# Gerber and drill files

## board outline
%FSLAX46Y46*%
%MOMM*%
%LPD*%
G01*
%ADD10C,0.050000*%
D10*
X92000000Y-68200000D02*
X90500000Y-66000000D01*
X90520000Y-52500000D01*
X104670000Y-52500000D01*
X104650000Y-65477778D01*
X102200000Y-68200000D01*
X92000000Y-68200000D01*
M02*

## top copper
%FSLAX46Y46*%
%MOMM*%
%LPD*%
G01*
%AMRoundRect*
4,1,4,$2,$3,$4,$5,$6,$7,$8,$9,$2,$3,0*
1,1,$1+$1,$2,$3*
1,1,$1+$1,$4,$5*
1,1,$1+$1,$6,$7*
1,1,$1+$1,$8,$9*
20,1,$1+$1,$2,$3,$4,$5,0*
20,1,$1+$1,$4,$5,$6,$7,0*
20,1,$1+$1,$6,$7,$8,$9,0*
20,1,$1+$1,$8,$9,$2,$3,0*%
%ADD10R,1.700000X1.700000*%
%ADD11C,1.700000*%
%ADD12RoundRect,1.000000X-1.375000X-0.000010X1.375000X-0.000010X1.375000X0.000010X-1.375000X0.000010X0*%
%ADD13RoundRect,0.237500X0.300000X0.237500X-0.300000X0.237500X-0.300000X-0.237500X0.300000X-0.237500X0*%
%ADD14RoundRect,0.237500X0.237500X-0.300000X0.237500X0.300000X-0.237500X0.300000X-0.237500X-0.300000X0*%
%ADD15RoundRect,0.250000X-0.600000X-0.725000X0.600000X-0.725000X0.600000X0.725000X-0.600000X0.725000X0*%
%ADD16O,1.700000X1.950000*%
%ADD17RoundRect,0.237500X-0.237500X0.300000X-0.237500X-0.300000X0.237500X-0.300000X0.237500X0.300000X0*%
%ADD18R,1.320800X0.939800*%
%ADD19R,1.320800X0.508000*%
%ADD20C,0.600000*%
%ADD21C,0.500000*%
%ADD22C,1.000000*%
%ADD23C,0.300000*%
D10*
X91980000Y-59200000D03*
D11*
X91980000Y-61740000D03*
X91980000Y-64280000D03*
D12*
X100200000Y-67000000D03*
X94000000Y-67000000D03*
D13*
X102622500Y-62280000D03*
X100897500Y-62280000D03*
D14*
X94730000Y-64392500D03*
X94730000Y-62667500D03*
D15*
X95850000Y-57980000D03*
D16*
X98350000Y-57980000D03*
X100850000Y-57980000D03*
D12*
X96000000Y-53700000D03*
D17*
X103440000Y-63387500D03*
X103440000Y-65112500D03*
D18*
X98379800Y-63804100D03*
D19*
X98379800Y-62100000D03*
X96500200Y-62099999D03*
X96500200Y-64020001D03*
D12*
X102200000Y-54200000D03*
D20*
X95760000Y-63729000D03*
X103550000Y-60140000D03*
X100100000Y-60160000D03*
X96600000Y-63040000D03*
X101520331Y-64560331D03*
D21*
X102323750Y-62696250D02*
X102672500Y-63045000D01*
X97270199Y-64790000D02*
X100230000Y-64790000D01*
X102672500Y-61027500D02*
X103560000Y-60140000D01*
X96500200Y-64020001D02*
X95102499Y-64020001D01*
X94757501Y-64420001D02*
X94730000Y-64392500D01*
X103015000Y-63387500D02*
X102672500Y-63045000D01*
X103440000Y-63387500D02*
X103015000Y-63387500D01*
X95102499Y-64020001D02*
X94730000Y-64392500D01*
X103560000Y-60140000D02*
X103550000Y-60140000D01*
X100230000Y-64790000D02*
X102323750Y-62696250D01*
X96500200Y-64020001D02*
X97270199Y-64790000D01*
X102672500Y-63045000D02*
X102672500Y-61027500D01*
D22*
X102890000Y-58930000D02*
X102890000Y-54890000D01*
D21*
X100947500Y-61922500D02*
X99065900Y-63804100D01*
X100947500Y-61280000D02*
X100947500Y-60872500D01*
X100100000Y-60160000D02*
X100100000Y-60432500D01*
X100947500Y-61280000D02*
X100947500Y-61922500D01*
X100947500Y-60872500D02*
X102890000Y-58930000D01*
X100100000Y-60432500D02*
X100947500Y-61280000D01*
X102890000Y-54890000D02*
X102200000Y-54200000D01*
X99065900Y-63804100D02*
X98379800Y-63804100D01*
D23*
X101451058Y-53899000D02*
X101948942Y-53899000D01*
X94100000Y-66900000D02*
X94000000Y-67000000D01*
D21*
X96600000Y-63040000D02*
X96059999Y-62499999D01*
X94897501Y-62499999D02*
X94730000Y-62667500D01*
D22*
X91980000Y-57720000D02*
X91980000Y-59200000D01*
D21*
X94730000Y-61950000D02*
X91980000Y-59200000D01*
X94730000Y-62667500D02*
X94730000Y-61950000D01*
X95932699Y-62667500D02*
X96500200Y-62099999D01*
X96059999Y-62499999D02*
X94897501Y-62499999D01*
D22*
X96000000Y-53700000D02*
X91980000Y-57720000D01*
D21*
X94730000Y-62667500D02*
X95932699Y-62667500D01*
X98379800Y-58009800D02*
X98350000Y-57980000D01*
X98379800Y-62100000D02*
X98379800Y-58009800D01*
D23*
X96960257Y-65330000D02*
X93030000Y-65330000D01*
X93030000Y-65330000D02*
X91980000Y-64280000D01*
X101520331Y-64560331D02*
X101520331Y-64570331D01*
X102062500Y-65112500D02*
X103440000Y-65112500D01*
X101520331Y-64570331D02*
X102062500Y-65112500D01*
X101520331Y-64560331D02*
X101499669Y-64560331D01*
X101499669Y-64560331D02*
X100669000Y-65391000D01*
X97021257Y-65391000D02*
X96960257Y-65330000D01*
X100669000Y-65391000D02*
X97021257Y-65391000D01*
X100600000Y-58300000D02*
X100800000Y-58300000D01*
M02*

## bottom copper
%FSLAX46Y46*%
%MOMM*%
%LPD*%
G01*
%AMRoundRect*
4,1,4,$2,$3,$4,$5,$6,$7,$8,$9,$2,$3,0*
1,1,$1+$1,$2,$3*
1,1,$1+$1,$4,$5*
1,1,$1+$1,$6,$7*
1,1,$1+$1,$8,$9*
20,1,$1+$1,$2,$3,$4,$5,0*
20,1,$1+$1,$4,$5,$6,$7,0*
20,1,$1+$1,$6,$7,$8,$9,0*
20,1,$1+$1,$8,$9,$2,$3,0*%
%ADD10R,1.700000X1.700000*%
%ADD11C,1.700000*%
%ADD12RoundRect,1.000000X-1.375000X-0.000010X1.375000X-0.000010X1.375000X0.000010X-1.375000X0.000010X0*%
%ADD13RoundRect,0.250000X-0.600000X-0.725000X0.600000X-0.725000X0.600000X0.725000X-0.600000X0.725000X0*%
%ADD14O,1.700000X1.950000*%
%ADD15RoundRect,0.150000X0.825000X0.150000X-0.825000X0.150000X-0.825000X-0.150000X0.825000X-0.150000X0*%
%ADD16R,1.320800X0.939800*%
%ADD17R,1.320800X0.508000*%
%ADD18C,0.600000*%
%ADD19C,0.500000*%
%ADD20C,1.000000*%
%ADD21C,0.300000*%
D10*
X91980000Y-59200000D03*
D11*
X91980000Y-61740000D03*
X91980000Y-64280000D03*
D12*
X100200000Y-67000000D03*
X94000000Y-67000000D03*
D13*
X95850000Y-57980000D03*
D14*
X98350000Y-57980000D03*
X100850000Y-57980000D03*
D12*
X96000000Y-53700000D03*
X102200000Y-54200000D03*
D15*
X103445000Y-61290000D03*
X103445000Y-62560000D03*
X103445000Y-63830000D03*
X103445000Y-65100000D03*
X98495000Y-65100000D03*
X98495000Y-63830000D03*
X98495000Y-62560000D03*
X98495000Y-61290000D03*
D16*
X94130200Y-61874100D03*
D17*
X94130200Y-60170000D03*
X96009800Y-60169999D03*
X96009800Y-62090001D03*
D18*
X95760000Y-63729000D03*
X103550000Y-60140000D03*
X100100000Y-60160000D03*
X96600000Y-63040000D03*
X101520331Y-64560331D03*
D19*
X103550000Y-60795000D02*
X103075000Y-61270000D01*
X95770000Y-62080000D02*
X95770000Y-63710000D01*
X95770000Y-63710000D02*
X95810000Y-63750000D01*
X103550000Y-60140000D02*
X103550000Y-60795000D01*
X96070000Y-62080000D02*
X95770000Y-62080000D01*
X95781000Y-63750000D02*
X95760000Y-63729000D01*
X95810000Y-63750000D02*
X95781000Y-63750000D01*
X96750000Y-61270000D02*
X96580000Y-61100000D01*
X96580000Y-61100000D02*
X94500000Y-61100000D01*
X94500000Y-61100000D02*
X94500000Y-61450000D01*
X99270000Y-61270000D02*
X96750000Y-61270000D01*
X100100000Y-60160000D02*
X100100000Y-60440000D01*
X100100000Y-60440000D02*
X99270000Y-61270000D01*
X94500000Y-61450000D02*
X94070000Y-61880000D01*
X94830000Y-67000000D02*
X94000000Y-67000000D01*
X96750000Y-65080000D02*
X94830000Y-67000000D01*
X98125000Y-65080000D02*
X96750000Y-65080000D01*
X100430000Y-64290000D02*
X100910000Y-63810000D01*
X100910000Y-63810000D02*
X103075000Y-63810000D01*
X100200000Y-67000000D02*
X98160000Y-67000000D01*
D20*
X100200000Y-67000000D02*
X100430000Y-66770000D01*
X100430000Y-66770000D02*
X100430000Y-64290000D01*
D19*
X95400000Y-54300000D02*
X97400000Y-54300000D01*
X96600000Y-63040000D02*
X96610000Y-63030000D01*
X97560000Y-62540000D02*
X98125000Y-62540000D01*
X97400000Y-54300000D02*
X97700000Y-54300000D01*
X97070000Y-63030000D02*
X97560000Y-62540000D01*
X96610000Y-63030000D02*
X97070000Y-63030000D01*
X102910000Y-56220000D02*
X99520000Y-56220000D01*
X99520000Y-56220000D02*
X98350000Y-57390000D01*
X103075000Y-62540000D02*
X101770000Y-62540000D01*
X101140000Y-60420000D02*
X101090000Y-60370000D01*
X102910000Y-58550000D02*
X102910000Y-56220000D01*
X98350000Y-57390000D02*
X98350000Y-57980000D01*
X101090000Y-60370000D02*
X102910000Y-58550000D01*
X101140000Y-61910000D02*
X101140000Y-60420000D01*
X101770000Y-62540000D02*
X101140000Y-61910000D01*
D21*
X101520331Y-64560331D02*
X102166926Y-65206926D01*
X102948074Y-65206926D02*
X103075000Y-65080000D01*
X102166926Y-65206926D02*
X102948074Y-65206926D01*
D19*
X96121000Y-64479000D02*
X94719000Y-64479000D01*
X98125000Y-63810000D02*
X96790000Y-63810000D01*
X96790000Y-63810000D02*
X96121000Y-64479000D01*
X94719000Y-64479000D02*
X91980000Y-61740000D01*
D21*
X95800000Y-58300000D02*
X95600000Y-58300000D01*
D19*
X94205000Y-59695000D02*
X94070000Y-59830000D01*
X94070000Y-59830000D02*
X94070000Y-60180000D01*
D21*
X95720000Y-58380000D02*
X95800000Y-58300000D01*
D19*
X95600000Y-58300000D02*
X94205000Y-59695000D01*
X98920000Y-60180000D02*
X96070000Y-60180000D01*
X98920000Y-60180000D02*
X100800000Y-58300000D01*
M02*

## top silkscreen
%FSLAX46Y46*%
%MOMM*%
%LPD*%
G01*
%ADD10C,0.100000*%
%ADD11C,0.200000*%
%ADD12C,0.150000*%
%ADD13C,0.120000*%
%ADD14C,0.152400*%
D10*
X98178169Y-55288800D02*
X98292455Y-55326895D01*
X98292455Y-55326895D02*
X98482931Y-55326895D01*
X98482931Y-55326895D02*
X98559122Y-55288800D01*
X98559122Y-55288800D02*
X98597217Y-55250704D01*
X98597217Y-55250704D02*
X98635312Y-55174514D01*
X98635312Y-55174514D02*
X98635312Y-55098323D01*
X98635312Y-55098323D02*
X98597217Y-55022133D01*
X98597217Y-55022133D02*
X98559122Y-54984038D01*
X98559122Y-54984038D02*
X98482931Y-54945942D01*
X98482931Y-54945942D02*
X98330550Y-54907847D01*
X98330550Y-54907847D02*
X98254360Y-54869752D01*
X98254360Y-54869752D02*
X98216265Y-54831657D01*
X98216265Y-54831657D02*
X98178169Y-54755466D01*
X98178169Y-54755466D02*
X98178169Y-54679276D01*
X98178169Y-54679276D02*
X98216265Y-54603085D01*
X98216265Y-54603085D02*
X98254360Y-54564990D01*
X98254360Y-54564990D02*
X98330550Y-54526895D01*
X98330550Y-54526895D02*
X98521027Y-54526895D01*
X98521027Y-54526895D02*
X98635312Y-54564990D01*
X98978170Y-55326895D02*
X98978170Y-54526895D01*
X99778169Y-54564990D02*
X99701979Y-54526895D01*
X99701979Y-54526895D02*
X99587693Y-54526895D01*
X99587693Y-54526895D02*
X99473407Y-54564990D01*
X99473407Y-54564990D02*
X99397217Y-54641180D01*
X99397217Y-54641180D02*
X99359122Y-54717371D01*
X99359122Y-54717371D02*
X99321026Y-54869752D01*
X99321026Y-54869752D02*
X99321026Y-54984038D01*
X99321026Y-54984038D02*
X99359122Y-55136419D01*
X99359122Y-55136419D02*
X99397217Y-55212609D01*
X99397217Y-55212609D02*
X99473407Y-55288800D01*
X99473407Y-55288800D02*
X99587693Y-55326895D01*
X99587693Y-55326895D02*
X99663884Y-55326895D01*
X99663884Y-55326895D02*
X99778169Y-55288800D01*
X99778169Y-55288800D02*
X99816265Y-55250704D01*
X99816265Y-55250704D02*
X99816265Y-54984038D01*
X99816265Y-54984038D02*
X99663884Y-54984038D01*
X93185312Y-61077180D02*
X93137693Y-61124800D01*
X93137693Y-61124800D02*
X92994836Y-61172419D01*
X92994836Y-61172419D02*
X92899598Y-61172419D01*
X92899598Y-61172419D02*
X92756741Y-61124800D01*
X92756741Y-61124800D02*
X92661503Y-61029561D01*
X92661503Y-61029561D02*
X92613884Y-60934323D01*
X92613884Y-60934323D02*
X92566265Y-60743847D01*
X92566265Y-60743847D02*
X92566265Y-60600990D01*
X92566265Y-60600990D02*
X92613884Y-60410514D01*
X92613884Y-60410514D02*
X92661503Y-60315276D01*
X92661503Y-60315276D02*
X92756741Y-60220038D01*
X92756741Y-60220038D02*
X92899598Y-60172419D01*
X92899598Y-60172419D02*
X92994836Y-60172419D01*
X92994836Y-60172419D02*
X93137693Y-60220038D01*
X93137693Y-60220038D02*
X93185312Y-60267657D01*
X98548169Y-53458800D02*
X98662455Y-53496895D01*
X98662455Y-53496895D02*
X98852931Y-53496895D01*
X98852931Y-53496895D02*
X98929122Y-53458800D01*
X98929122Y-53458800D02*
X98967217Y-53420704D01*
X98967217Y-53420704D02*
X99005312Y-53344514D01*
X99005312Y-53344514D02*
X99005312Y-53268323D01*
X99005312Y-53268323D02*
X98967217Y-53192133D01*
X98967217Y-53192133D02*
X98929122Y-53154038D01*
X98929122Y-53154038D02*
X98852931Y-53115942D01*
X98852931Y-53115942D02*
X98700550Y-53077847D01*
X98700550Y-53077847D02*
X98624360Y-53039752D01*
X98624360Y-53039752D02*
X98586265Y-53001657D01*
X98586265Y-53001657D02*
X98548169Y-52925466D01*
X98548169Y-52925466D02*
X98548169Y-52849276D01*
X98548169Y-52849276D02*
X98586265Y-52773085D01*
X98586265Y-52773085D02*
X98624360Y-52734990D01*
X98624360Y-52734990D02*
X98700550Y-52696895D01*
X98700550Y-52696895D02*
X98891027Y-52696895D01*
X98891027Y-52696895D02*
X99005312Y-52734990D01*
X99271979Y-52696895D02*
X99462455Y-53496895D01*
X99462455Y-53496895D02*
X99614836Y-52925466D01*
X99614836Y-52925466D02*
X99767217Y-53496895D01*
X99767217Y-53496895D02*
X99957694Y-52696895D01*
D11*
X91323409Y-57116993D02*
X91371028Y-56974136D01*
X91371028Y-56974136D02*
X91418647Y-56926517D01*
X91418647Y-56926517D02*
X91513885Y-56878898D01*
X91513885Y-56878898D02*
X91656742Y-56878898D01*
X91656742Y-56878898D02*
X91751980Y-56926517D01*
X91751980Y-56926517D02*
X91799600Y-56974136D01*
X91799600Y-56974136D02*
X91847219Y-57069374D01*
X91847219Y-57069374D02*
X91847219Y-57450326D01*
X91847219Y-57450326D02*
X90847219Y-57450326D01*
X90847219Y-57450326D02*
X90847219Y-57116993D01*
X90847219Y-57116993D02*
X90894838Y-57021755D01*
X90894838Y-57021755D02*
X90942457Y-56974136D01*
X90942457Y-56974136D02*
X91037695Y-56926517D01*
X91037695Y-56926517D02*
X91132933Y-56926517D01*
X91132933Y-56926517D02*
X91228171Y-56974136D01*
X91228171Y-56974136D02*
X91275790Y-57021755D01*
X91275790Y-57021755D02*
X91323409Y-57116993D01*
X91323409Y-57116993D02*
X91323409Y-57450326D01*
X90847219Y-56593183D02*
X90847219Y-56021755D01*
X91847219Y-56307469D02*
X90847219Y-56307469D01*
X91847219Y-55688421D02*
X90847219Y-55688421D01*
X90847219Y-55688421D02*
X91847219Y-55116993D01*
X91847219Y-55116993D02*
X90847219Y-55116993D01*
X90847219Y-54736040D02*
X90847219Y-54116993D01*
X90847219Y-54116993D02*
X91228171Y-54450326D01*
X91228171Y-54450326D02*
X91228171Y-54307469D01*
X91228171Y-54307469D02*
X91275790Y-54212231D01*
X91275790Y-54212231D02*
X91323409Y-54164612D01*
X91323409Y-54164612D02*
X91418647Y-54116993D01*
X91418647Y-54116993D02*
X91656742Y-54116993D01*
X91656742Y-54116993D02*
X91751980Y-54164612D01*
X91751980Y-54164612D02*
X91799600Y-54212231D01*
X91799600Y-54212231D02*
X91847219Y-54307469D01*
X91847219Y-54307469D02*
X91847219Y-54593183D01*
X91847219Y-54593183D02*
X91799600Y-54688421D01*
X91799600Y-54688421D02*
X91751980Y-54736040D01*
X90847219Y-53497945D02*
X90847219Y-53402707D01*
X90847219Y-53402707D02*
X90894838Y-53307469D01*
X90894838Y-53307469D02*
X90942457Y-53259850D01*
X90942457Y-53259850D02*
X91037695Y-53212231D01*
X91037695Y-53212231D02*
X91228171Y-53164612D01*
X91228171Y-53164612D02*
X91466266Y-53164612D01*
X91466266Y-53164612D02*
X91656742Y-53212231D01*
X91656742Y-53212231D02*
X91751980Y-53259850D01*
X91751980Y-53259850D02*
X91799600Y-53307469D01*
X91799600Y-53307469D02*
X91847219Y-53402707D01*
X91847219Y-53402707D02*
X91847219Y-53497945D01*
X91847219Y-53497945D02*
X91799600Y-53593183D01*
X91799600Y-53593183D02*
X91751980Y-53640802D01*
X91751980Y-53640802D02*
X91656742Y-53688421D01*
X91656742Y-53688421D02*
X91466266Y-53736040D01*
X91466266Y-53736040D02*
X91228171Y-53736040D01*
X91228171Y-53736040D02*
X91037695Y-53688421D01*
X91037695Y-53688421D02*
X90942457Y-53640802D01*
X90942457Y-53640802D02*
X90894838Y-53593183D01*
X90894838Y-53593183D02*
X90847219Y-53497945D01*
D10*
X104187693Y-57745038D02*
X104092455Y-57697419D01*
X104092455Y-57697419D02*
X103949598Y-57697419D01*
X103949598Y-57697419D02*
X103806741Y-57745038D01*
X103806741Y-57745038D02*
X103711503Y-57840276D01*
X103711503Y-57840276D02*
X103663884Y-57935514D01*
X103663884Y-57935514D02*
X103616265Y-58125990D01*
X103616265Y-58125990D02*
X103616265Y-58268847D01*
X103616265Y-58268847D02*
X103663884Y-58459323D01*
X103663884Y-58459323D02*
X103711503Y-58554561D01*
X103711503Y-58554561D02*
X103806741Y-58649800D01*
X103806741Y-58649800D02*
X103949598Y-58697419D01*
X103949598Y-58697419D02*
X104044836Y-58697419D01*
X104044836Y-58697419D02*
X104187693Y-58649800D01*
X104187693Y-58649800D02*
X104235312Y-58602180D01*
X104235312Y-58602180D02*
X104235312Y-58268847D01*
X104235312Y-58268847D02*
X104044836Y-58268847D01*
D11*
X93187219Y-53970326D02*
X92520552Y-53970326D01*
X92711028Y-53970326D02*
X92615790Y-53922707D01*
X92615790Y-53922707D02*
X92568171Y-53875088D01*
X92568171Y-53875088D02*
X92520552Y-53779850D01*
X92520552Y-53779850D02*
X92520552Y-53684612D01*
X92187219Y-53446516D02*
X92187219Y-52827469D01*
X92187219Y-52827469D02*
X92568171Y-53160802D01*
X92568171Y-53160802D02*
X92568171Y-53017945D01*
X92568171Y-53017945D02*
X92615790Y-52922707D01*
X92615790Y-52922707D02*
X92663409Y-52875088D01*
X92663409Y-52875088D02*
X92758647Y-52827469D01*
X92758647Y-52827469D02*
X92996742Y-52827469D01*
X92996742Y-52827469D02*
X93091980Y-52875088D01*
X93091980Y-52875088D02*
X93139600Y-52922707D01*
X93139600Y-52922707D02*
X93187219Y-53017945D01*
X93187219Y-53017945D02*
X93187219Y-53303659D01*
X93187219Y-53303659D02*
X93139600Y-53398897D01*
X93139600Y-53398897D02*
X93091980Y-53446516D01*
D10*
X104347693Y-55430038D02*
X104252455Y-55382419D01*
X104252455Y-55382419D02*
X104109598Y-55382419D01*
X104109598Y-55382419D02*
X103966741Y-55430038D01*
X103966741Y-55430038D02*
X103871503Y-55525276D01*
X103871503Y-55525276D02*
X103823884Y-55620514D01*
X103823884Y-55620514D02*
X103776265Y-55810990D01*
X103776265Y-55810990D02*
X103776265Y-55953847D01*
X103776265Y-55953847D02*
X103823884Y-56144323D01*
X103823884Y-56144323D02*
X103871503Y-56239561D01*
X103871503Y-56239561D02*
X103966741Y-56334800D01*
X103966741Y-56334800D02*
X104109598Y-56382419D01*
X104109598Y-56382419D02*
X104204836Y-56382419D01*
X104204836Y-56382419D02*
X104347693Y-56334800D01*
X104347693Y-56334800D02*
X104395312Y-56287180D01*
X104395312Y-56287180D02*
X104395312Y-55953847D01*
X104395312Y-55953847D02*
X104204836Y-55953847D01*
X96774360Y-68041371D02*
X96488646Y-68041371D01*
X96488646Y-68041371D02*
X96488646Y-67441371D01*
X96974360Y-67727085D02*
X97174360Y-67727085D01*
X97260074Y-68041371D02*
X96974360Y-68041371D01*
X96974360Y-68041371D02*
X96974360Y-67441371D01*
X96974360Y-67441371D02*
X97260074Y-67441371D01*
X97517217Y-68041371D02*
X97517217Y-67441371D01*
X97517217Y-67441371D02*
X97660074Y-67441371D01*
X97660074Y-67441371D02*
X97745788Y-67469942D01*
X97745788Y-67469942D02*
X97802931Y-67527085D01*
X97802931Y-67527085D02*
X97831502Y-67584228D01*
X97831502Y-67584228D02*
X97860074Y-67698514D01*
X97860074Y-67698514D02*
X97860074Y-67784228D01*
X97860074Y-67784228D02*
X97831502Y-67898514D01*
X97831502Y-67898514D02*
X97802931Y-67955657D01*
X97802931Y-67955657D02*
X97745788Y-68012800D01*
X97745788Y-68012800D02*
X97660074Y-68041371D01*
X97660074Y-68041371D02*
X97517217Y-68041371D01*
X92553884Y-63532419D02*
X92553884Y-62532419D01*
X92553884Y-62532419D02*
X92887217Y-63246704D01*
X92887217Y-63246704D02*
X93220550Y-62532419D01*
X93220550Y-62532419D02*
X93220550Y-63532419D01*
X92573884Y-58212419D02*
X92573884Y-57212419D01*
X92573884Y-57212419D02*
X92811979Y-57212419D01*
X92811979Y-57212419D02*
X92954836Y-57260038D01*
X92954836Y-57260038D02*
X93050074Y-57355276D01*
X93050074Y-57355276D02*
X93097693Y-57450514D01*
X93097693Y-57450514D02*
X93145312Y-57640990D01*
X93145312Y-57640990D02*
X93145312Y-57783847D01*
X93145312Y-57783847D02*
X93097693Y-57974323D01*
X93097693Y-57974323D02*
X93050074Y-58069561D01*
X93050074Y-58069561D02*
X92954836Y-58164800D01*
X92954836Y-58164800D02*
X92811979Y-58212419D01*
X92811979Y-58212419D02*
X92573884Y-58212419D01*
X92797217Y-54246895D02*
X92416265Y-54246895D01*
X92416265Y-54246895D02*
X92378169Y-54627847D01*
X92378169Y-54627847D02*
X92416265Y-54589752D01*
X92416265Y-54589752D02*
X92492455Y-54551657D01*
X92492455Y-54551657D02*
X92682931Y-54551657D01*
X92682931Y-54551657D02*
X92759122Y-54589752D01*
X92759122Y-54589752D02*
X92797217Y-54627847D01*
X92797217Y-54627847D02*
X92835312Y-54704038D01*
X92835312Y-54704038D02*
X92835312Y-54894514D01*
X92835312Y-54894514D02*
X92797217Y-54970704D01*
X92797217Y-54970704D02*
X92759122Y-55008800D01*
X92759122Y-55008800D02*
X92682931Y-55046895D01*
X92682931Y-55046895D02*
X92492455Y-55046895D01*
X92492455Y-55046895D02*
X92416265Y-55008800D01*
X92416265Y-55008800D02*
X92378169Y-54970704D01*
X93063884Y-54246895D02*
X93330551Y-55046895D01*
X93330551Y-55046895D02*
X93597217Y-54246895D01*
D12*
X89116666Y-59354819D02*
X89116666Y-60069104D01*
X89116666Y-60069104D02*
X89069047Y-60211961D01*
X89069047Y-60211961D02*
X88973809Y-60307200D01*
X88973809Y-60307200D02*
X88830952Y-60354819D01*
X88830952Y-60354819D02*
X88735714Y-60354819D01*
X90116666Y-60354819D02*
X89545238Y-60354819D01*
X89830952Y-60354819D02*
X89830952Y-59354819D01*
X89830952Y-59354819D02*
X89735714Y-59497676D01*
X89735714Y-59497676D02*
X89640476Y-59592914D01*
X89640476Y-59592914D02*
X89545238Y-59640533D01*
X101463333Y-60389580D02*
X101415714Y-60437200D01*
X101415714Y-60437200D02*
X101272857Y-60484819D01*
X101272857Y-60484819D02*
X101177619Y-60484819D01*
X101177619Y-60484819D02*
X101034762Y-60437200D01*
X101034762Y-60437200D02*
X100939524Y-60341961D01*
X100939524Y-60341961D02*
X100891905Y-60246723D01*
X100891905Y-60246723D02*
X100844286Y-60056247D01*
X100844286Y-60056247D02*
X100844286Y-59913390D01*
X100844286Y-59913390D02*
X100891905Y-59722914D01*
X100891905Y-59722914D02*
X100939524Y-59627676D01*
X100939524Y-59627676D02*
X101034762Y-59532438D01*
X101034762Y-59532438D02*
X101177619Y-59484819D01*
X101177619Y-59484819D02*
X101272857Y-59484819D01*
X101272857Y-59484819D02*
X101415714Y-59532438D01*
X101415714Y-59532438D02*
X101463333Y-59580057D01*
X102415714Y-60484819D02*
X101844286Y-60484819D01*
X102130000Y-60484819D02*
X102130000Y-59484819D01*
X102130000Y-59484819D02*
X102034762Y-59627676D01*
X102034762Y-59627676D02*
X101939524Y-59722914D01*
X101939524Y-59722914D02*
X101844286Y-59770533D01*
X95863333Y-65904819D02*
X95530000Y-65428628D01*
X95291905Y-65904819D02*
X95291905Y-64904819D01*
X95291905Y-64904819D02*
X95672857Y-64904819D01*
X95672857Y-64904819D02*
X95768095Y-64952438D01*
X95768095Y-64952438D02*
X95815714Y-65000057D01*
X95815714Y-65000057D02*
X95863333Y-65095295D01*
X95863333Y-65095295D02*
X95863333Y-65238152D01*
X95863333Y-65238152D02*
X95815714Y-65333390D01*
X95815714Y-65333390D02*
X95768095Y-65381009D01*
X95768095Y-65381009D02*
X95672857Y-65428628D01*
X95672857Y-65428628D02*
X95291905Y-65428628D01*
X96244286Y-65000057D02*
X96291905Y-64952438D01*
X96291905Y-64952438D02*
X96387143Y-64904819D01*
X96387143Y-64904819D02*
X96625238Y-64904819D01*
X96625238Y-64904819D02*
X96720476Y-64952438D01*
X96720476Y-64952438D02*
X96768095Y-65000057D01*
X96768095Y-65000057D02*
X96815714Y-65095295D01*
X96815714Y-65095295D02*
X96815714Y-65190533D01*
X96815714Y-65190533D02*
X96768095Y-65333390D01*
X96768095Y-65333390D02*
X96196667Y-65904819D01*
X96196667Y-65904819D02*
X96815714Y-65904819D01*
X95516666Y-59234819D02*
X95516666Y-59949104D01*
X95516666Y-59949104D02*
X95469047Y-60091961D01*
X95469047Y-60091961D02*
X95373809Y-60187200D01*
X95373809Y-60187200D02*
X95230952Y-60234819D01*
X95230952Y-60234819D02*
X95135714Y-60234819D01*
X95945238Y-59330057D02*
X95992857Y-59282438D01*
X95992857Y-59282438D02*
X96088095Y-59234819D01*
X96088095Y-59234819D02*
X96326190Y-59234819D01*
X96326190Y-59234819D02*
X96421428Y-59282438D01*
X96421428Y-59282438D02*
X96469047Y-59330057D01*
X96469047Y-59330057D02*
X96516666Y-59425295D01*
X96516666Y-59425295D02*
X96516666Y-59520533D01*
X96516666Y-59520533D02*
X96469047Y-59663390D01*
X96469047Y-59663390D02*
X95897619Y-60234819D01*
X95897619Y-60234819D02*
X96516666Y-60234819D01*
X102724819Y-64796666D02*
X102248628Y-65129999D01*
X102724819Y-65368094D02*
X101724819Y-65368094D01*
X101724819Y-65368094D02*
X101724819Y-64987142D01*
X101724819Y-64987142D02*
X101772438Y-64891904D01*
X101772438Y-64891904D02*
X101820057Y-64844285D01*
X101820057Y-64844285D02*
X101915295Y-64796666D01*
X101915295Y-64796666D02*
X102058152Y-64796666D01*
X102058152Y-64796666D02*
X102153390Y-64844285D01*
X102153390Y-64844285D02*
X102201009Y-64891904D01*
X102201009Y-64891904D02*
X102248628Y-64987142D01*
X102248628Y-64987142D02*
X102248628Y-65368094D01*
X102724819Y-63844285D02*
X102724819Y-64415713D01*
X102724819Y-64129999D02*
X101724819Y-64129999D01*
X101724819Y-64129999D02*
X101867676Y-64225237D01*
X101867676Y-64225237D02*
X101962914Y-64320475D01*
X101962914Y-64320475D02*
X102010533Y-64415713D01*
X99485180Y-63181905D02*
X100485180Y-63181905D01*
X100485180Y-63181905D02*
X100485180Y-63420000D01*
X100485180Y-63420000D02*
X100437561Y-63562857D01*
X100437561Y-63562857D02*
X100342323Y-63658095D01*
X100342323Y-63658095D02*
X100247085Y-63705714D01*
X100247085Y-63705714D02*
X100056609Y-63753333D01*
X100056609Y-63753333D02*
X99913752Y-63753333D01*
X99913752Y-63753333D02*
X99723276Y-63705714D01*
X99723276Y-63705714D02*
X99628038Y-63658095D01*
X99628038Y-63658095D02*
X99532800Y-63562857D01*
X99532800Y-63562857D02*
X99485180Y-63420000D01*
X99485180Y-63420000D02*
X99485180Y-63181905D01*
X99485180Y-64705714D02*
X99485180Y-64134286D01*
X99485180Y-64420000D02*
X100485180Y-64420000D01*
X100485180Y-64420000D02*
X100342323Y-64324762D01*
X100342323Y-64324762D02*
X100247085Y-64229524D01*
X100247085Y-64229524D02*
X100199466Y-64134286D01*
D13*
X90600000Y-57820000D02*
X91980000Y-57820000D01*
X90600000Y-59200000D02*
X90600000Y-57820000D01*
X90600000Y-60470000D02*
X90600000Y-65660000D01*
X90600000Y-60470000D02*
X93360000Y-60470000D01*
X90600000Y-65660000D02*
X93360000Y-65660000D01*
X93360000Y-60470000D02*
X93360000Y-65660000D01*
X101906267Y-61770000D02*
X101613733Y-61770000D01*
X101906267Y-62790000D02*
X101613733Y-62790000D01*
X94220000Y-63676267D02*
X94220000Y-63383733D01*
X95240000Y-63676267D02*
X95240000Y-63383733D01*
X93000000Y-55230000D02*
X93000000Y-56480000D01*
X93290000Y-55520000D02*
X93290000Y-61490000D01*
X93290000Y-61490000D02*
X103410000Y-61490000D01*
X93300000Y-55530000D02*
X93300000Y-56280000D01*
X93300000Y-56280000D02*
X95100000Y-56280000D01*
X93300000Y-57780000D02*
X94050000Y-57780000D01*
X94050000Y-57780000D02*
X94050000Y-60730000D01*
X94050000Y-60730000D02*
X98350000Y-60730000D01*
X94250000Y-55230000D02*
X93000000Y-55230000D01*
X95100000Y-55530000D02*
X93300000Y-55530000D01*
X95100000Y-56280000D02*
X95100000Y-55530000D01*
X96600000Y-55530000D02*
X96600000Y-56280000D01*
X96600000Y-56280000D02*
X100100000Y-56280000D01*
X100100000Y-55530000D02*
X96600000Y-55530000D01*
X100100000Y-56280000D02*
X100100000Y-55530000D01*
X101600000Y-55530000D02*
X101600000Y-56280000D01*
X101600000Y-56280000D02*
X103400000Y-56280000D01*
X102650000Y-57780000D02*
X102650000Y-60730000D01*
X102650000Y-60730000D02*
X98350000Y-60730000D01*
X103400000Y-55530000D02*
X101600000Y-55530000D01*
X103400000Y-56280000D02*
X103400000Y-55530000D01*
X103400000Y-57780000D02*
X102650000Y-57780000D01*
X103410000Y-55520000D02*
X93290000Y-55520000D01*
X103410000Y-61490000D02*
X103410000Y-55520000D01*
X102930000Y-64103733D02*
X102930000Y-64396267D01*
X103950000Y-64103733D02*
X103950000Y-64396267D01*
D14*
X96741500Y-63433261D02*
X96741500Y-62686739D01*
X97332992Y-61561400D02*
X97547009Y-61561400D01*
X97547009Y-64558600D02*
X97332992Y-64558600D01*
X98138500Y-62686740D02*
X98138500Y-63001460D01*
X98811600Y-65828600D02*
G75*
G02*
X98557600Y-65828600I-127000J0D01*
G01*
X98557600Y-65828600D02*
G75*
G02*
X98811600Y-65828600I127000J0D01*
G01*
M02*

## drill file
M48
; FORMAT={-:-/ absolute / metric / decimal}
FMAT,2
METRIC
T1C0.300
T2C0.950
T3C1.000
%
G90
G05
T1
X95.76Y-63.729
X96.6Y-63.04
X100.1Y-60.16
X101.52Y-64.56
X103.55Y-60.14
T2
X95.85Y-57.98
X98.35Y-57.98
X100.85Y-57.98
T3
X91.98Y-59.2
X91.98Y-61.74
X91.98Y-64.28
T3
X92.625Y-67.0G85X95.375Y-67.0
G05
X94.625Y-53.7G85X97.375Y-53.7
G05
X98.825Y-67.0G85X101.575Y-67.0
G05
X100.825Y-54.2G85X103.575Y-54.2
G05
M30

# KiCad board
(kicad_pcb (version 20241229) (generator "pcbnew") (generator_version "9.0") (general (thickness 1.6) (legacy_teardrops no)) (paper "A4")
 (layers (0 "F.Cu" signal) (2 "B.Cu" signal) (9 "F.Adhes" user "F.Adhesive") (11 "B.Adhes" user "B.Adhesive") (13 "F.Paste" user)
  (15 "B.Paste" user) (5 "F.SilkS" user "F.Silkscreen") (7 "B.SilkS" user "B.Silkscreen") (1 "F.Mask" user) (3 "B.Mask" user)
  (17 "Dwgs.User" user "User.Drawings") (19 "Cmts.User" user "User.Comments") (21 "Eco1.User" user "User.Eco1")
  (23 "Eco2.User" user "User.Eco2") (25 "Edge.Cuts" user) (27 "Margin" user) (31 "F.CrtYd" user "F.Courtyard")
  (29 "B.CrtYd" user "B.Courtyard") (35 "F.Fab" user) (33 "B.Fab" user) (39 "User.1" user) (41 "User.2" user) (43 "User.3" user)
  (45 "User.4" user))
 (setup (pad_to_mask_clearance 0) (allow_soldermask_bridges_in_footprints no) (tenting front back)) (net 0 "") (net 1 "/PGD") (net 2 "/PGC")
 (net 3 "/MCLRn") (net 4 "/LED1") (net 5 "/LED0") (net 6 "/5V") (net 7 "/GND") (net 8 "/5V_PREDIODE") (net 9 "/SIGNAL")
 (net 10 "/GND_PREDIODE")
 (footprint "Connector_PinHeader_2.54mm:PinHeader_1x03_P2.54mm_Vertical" (layer "F.Cu") (at 91.98 59.2)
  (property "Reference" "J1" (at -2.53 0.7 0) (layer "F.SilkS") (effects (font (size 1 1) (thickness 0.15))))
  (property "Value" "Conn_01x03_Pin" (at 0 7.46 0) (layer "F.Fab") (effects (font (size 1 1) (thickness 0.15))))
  (fp_line (start -1.38 -1.38) (end 0 -1.38) (stroke (width 0.12) (type solid)) (layer "F.SilkS"))
  (fp_line (start -1.38 0) (end -1.38 -1.38) (stroke (width 0.12) (type solid)) (layer "F.SilkS"))
  (fp_line (start -1.38 1.27) (end -1.38 6.46) (stroke (width 0.12) (type solid)) (layer "F.SilkS"))
  (fp_line (start -1.38 1.27) (end 1.38 1.27) (stroke (width 0.12) (type solid)) (layer "F.SilkS"))
  (fp_line (start -1.38 6.46) (end 1.38 6.46) (stroke (width 0.12) (type solid)) (layer "F.SilkS"))
  (fp_line (start 1.38 1.27) (end 1.38 6.46) (stroke (width 0.12) (type solid)) (layer "F.SilkS"))
  (pad "1" thru_hole rect (at 0 0) (size 1.7 1.7) (drill 1) (layers "*.Cu" "*.Mask") (remove_unused_layers no) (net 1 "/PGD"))
  (pad "2" thru_hole circle (at 0 2.54) (size 1.7 1.7) (drill 1) (layers "*.Cu" "*.Mask") (remove_unused_layers no) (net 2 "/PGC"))
  (pad "3" thru_hole circle (at 0 5.08) (size 1.7 1.7) (drill 1) (layers "*.Cu" "*.Mask") (remove_unused_layers no) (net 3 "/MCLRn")))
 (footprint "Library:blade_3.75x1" (layer "F.Cu") (at 100.2 67)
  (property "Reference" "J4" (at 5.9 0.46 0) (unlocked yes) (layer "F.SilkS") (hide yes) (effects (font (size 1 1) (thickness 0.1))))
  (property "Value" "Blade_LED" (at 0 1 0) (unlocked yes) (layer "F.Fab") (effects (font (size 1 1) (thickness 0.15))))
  (pad "1" thru_hole roundrect (at 0 0) (size 4.75 2) (drill oval 3.75 1) (layers "*.Cu" "*.Mask") (remove_unused_layers no)
   (roundrect_rratio 0.5) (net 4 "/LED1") (thermal_bridge_angle 45)))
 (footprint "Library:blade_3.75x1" (layer "F.Cu") (at 94 67)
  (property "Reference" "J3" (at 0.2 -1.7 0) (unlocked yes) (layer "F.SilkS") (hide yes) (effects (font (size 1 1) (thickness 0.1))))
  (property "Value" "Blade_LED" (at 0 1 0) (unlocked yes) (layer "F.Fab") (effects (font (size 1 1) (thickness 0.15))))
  (pad "1" thru_hole roundrect (at 0 0) (size 4.75 2) (drill oval 3.75 1) (layers "*.Cu" "*.Mask") (remove_unused_layers no)
   (roundrect_rratio 0.5) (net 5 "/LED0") (thermal_bridge_angle 45)))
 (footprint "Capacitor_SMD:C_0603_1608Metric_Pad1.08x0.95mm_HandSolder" (layer "F.Cu") (at 101.76 62.28 180)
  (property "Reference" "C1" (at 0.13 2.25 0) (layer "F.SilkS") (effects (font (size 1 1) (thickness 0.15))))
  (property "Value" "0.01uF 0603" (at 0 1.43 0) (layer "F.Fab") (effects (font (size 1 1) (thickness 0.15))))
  (fp_line (start -0.146267 0.51) (end 0.146267 0.51) (stroke (width 0.12) (type solid)) (layer "F.SilkS"))
  (fp_line (start -0.146267 -0.51) (end 0.146267 -0.51) (stroke (width 0.12) (type solid)) (layer "F.SilkS"))
  (pad "1" smd roundrect (at -0.8625 0 180) (size 1.075 0.95) (layers "F.Cu" "F.Mask" "F.Paste") (roundrect_rratio 0.25) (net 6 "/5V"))
  (pad "2" smd roundrect (at 0.8625 0 180) (size 1.075 0.95) (layers "F.Cu" "F.Mask" "F.Paste") (roundrect_rratio 0.25) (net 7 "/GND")))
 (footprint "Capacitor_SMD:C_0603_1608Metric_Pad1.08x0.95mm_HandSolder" (layer "F.Cu") (at 94.73 63.53 90)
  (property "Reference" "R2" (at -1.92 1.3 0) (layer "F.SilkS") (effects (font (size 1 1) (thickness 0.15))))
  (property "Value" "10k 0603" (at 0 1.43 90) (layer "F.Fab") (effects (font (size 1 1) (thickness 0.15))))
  (fp_line (start -0.146267 -0.51) (end 0.146267 -0.51) (stroke (width 0.12) (type solid)) (layer "F.SilkS"))
  (fp_line (start -0.146267 0.51) (end 0.146267 0.51) (stroke (width 0.12) (type solid)) (layer "F.SilkS"))
  (pad "1" smd roundrect (at -0.8625 0 90) (size 1.075 0.95) (layers "F.Cu" "F.Mask" "F.Paste") (roundrect_rratio 0.25) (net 6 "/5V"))
  (pad "2" smd roundrect (at 0.8625 0 90) (size 1.075 0.95) (layers "F.Cu" "F.Mask" "F.Paste") (roundrect_rratio 0.25) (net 1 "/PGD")))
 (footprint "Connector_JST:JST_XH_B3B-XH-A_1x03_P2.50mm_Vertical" (layer "F.Cu") (at 95.85 57.98)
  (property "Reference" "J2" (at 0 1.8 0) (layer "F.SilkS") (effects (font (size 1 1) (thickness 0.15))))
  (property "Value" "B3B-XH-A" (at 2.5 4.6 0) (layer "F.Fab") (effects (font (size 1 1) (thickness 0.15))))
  (fp_line (start -2.85 -2.75) (end -2.85 -1.5) (stroke (width 0.12) (type solid)) (layer "F.SilkS"))
  (fp_line (start -2.56 -2.46) (end -2.56 3.51) (stroke (width 0.12) (type solid)) (layer "F.SilkS"))
  (fp_line (start -2.56 3.51) (end 7.56 3.51) (stroke (width 0.12) (type solid)) (layer "F.SilkS"))
  (fp_line (start -2.55 -2.45) (end -2.55 -1.7) (stroke (width 0.12) (type solid)) (layer "F.SilkS"))
  (fp_line (start -2.55 -1.7) (end -0.75 -1.7) (stroke (width 0.12) (type solid)) (layer "F.SilkS"))
  (fp_line (start -2.55 -0.2) (end -1.8 -0.2) (stroke (width 0.12) (type solid)) (layer "F.SilkS"))
  (fp_line (start -1.8 -0.2) (end -1.8 2.75) (stroke (width 0.12) (type solid)) (layer "F.SilkS"))
  (fp_line (start -1.8 2.75) (end 2.5 2.75) (stroke (width 0.12) (type solid)) (layer "F.SilkS"))
  (fp_line (start -1.6 -2.75) (end -2.85 -2.75) (stroke (width 0.12) (type solid)) (layer "F.SilkS"))
  (fp_line (start -0.75 -2.45) (end -2.55 -2.45) (stroke (width 0.12) (type solid)) (layer "F.SilkS"))
  (fp_line (start -0.75 -1.7) (end -0.75 -2.45) (stroke (width 0.12) (type solid)) (layer "F.SilkS"))
  (fp_line (start 0.75 -2.45) (end 0.75 -1.7) (stroke (width 0.12) (type solid)) (layer "F.SilkS"))
  (fp_line (start 0.75 -1.7) (end 4.25 -1.7) (stroke (width 0.12) (type solid)) (layer "F.SilkS"))
  (fp_line (start 4.25 -2.45) (end 0.75 -2.45) (stroke (width 0.12) (type solid)) (layer "F.SilkS"))
  (fp_line (start 4.25 -1.7) (end 4.25 -2.45) (stroke (width 0.12) (type solid)) (layer "F.SilkS"))
  (fp_line (start 5.75 -2.45) (end 5.75 -1.7) (stroke (width 0.12) (type solid)) (layer "F.SilkS"))
  (fp_line (start 5.75 -1.7) (end 7.55 -1.7) (stroke (width 0.12) (type solid)) (layer "F.SilkS"))
  (fp_line (start 6.8 -0.2) (end 6.8 2.75) (stroke (width 0.12) (type solid)) (layer "F.SilkS"))
  (fp_line (start 6.8 2.75) (end 2.5 2.75) (stroke (width 0.12) (type solid)) (layer "F.SilkS"))
  (fp_line (start 7.55 -2.45) (end 5.75 -2.45) (stroke (width 0.12) (type solid)) (layer "F.SilkS"))
  (fp_line (start 7.55 -1.7) (end 7.55 -2.45) (stroke (width 0.12) (type solid)) (layer "F.SilkS"))
  (fp_line (start 7.55 -0.2) (end 6.8 -0.2) (stroke (width 0.12) (type solid)) (layer "F.SilkS"))
  (fp_line (start 7.56 -2.46) (end -2.56 -2.46) (stroke (width 0.12) (type solid)) (layer "F.SilkS"))
  (fp_line (start 7.56 3.51) (end 7.56 -2.46) (stroke (width 0.12) (type solid)) (layer "F.SilkS"))
  (pad "1" thru_hole roundrect (at 0 0) (size 1.7 1.95) (drill 0.95) (layers "*.Cu" "*.Mask") (remove_unused_layers no)
   (roundrect_rratio 0.147059) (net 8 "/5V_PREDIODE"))
  (pad "2" thru_hole oval (at 2.5 0) (size 1.7 1.95) (drill 0.95) (layers "*.Cu" "*.Mask") (remove_unused_layers no) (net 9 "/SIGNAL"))
  (pad "3" thru_hole oval (at 5 0) (size 1.7 1.95) (drill 0.95) (layers "*.Cu" "*.Mask") (remove_unused_layers no) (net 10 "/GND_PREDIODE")))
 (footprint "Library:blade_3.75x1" (layer "F.Cu") (at 95.4 54.3)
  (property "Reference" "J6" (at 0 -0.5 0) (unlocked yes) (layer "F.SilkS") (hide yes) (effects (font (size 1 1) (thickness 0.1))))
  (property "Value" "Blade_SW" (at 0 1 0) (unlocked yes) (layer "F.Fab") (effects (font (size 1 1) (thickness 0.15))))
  (pad "1" thru_hole roundrect (at 0.6 -0.6) (size 4.75 2) (drill oval 3.75 1) (layers "*.Cu" "*.Mask") (remove_unused_layers no)
   (roundrect_rratio 0.5) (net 1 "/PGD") (thermal_bridge_angle 45)))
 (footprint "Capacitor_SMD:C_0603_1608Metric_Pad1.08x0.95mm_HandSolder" (layer "F.Cu") (at 103.44 64.25 -90)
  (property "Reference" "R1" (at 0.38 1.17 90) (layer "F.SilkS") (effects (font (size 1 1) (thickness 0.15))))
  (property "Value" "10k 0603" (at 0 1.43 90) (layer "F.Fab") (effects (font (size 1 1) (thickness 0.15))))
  (fp_line (start -0.146267 0.51) (end 0.146267 0.51) (stroke (width 0.12) (type solid)) (layer "F.SilkS"))
  (fp_line (start -0.146267 -0.51) (end 0.146267 -0.51) (stroke (width 0.12) (type solid)) (layer "F.SilkS"))
  (pad "1" smd roundrect (at -0.8625 0 270) (size 1.075 0.95) (layers "F.Cu" "F.Mask" "F.Paste") (roundrect_rratio 0.25) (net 6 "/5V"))
  (pad "2" smd roundrect (at 0.8625 0 270) (size 1.075 0.95) (layers "F.Cu" "F.Mask" "F.Paste") (roundrect_rratio 0.25) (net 3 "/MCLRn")))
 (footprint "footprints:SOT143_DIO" (layer "F.Cu") (at 97.44 63.06 90)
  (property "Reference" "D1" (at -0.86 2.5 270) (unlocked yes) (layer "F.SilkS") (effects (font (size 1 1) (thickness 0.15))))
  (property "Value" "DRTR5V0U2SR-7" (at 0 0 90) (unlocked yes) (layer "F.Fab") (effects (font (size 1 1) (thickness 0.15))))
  (fp_line (start -0.373261 -0.6985) (end 0.373261 -0.6985) (stroke (width 0.1524) (type solid)) (layer "F.SilkS"))
  (fp_line (start 1.4986 -0.107008) (end 1.4986 0.107009) (stroke (width 0.1524) (type solid)) (layer "F.SilkS"))
  (fp_line (start -1.4986 0.107009) (end -1.4986 -0.107008) (stroke (width 0.1524) (type solid)) (layer "F.SilkS"))
  (fp_line (start 0.37326 0.6985) (end 0.05854 0.6985) (stroke (width 0.1524) (type solid)) (layer "F.SilkS"))
  (fp_circle (center -2.7686 1.2446) (end -2.6416 1.2446) (stroke (width 0.1524) (type solid)) (fill no) (layer "F.SilkS"))
  (pad "1" smd rect (at -0.7441 0.9398 90) (size 0.9398 1.3208) (layers "F.Cu" "F.Mask" "F.Paste") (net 7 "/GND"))
  (pad "2" smd rect (at 0.96 0.9398 90) (size 0.508 1.3208) (layers "F.Cu" "F.Mask" "F.Paste") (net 9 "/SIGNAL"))
  (pad "3" smd rect (at 0.960001 -0.9398 90) (size 0.508 1.3208) (layers "F.Cu" "F.Mask" "F.Paste") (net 1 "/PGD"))
  (pad "4" smd rect (at -0.960001 -0.9398 90) (size 0.508 1.3208) (layers "F.Cu" "F.Mask" "F.Paste") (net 6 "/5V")))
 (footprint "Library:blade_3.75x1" (layer "F.Cu") (at 101.7 55.5)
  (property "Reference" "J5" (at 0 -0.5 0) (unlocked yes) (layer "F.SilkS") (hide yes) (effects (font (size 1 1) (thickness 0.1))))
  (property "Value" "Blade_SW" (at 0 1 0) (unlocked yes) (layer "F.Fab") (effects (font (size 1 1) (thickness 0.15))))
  (pad "1" thru_hole roundrect (at 0.5 -1.3) (size 4.75 2) (drill oval 3.75 1) (layers "*.Cu" "*.Mask") (remove_unused_layers no)
   (roundrect_rratio 0.5) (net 7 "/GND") (thermal_bridge_angle 45)))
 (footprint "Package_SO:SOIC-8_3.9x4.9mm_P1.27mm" (layer "B.Cu") (at 100.97 63.195 180)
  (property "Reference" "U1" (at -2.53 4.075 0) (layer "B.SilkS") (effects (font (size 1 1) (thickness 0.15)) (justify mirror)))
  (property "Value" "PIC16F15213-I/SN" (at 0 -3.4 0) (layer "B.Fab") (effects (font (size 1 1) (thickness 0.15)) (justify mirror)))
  (pad "1" smd roundrect (at -2.475 1.905 180) (size 1.95 0.6) (layers "B.Cu" "B.Mask" "B.Paste") (roundrect_rratio 0.25) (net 6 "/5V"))
  (pad "2" smd roundrect (at -2.475 0.635 180) (size 1.95 0.6) (layers "B.Cu" "B.Mask" "B.Paste") (roundrect_rratio 0.25) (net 9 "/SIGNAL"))
  (pad "3" smd roundrect (at -2.475 -0.635 180) (size 1.95 0.6) (layers "B.Cu" "B.Mask" "B.Paste") (roundrect_rratio 0.25) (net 4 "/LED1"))
  (pad "4" smd roundrect (at -2.475 -1.905 180) (size 1.95 0.6) (layers "B.Cu" "B.Mask" "B.Paste") (roundrect_rratio 0.25) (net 3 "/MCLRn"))
  (pad "5" smd roundrect (at 2.475 -1.905 180) (size 1.95 0.6) (layers "B.Cu" "B.Mask" "B.Paste") (roundrect_rratio 0.25) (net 5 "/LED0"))
  (pad "6" smd roundrect (at 2.475 -0.635 180) (size 1.95 0.6) (layers "B.Cu" "B.Mask" "B.Paste") (roundrect_rratio 0.25) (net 2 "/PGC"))
  (pad "7" smd roundrect (at 2.475 0.635 180) (size 1.95 0.6) (layers "B.Cu" "B.Mask" "B.Paste") (roundrect_rratio 0.25) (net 1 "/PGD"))
  (pad "8" smd roundrect (at 2.475 1.905 180) (size 1.95 0.6) (layers "B.Cu" "B.Mask" "B.Paste") (roundrect_rratio 0.25) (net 7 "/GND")))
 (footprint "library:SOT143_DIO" (layer "B.Cu") (at 95.07 61.13 90)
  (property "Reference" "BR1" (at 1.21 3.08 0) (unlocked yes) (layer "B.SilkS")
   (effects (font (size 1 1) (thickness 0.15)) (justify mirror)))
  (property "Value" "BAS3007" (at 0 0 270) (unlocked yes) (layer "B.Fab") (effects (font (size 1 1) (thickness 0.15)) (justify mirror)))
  (pad "1" smd rect (at -0.7441 -0.9398 90) (size 0.9398 1.3208) (layers "B.Cu" "B.Mask" "B.Paste") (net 7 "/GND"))
  (pad "2" smd rect (at 0.96 -0.9398 90) (size 0.508 1.3208) (layers "B.Cu" "B.Mask" "B.Paste") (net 8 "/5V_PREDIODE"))
  (pad "3" smd rect (at 0.960001 0.9398 90) (size 0.508 1.3208) (layers "B.Cu" "B.Mask" "B.Paste") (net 10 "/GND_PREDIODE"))
  (pad "4" smd rect (at -0.960001 0.9398 90) (size 0.508 1.3208) (layers "B.Cu" "B.Mask" "B.Paste") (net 6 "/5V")))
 (gr_poly
  (pts (xy 92 68.2) (xy 90.5 66) (xy 90.52 52.5) (xy 104.67 52.5) (xy 104.65 65.477778) (xy 102.2 68.2)) (stroke (width 0.05) (type solid))
  (fill no) (layer "Edge.Cuts"))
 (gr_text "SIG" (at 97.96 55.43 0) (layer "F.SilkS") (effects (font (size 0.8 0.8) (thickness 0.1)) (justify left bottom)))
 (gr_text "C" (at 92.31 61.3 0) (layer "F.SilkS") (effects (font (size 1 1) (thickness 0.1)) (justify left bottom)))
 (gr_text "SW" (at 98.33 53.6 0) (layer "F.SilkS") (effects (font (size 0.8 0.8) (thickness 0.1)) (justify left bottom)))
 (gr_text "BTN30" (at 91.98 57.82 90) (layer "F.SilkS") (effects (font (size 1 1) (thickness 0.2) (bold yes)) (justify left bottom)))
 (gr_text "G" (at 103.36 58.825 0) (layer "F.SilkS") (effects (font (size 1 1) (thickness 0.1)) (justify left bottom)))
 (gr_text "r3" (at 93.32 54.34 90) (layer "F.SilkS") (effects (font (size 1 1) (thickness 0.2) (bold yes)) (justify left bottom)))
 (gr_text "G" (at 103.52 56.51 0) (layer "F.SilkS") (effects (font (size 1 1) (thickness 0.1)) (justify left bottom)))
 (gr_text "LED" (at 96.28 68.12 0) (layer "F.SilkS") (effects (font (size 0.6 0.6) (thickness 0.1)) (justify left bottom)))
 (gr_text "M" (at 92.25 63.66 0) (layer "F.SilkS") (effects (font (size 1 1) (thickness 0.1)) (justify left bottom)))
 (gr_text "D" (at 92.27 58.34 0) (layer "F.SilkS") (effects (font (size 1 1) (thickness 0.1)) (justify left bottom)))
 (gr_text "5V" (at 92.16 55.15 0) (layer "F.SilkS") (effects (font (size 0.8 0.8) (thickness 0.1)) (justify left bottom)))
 (segment (start 102.32375 62.69625) (end 102.6725 63.045) (width 0.5) (layer "F.Cu") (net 6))
 (segment (start 97.270199 64.79) (end 100.23 64.79) (width 0.5) (layer "F.Cu") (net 6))
 (segment (start 102.6725 61.0275) (end 103.56 60.14) (width 0.5) (layer "F.Cu") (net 6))
 (segment (start 96.5002 64.020001) (end 95.102499 64.020001) (width 0.5) (layer "F.Cu") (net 6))
 (segment (start 94.757501 64.420001) (end 94.73 64.3925) (width 0.5) (layer "F.Cu") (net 6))
 (segment (start 103.015 63.3875) (end 102.6725 63.045) (width 0.5) (layer "F.Cu") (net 6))
 (segment (start 103.44 63.3875) (end 103.015 63.3875) (width 0.5) (layer "F.Cu") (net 6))
 (segment (start 95.102499 64.020001) (end 94.73 64.3925) (width 0.5) (layer "F.Cu") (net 6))
 (segment (start 103.56 60.14) (end 103.55 60.14) (width 0.5) (layer "F.Cu") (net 6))
 (segment (start 100.23 64.79) (end 102.32375 62.69625) (width 0.5) (layer "F.Cu") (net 6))
 (segment (start 96.5002 64.020001) (end 97.270199 64.79) (width 0.5) (layer "F.Cu") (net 6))
 (segment (start 102.6725 63.045) (end 102.6725 61.0275) (width 0.5) (layer "F.Cu") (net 6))
 (via (at 95.76 63.729) (size 0.6) (drill 0.3) (layers "F.Cu" "B.Cu") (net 6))
 (via (at 103.55 60.14) (size 0.6) (drill 0.3) (layers "F.Cu" "B.Cu") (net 6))
 (segment (start 103.55 60.795) (end 103.075 61.27) (width 0.5) (layer "B.Cu") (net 6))
 (segment (start 95.77 62.08) (end 95.77 63.71) (width 0.5) (layer "B.Cu") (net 6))
 (segment (start 95.77 63.71) (end 95.81 63.75) (width 0.5) (layer "B.Cu") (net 6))
 (segment (start 103.55 60.14) (end 103.55 60.795) (width 0.5) (layer "B.Cu") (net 6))
 (segment (start 96.07 62.08) (end 95.77 62.08) (width 0.5) (layer "B.Cu") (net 6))
 (segment (start 95.781 63.75) (end 95.76 63.729) (width 0.5) (layer "B.Cu") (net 6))
 (segment (start 95.81 63.75) (end 95.781 63.75) (width 0.5) (layer "B.Cu") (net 6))
 (segment (start 102.89 58.93) (end 102.89 54.89) (width 1) (layer "F.Cu") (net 7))
 (segment (start 100.9475 61.9225) (end 99.0659 63.8041) (width 0.5) (layer "F.Cu") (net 7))
 (segment (start 100.9475 61.28) (end 100.9475 60.8725) (width 0.5) (layer "F.Cu") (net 7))
 (segment (start 100.1 60.16) (end 100.1 60.4325) (width 0.5) (layer "F.Cu") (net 7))
 (segment (start 100.9475 61.28) (end 100.9475 61.9225) (width 0.5) (layer "F.Cu") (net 7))
 (segment (start 100.9475 60.8725) (end 102.89 58.93) (width 0.5) (layer "F.Cu") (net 7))
 (segment (start 100.1 60.4325) (end 100.9475 61.28) (width 0.5) (layer "F.Cu") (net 7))
 (segment (start 102.89 54.89) (end 102.2 54.2) (width 0.5) (layer "F.Cu") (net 7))
 (segment (start 99.0659 63.8041) (end 98.3798 63.8041) (width 0.5) (layer "F.Cu") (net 7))
 (segment (start 101.451058 53.899) (end 101.948942 53.899) (width 0.3) (layer "F.Cu") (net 7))
 (via (at 100.1 60.16) (size 0.6) (drill 0.3) (layers "F.Cu" "B.Cu") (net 7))
 (segment (start 96.75 61.27) (end 96.58 61.1) (width 0.5) (layer "B.Cu") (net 7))
 (segment (start 96.58 61.1) (end 94.5 61.1) (width 0.5) (layer "B.Cu") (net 7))
 (segment (start 94.5 61.1) (end 94.5 61.45) (width 0.5) (layer "B.Cu") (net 7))
 (segment (start 99.27 61.27) (end 96.75 61.27) (width 0.5) (layer "B.Cu") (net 7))
 (segment (start 100.1 60.16) (end 100.1 60.44) (width 0.5) (layer "B.Cu") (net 7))
 (segment (start 100.1 60.44) (end 99.27 61.27) (width 0.5) (layer "B.Cu") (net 7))
 (segment (start 94.5 61.45) (end 94.07 61.88) (width 0.5) (layer "B.Cu") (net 7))
 (segment (start 94.1 66.9) (end 94 67) (width 0.3) (layer "F.Cu") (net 5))
 (segment (start 94.83 67) (end 94 67) (width 0.5) (layer "B.Cu") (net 5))
 (segment (start 96.75 65.08) (end 94.83 67) (width 0.5) (layer "B.Cu") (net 5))
 (segment (start 98.125 65.08) (end 96.75 65.08) (width 0.5) (layer "B.Cu") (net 5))
 (segment (start 100.43 64.29) (end 100.91 63.81) (width 0.5) (layer "B.Cu") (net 4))
 (segment (start 100.91 63.81) (end 103.075 63.81) (width 0.5) (layer "B.Cu") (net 4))
 (segment (start 100.2 67) (end 98.16 67) (width 0.5) (layer "B.Cu") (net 4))
 (segment (start 100.2 67) (end 100.43 66.77) (width 1) (layer "B.Cu") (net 4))
 (segment (start 100.43 66.77) (end 100.43 64.29) (width 1) (layer "B.Cu") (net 4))
 (segment (start 96.6 63.04) (end 96.059999 62.499999) (width 0.5) (layer "F.Cu") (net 1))
 (segment (start 94.897501 62.499999) (end 94.73 62.6675) (width 0.5) (layer "F.Cu") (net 1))
 (segment (start 91.98 57.72) (end 91.98 59.2) (width 1) (layer "F.Cu") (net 1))
 (segment (start 94.73 61.95) (end 91.98 59.2) (width 0.5) (layer "F.Cu") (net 1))
 (segment (start 94.73 62.6675) (end 94.73 61.95) (width 0.5) (layer "F.Cu") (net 1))
 (segment (start 95.932699 62.6675) (end 96.5002 62.099999) (width 0.5) (layer "F.Cu") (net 1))
 (segment (start 96.059999 62.499999) (end 94.897501 62.499999) (width 0.5) (layer "F.Cu") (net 1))
 (segment (start 96 53.7) (end 91.98 57.72) (width 1) (layer "F.Cu") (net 1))
 (segment (start 94.73 62.6675) (end 95.932699 62.6675) (width 0.5) (layer "F.Cu") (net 1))
 (via (at 96.6 63.04) (size 0.6) (drill 0.3) (layers "F.Cu" "B.Cu") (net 1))
 (segment (start 95.4 54.3) (end 97.4 54.3) (width 0.5) (layer "B.Cu") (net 1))
 (segment (start 96.6 63.04) (end 96.61 63.03) (width 0.5) (layer "B.Cu") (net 1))
 (segment (start 97.56 62.54) (end 98.125 62.54) (width 0.5) (layer "B.Cu") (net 1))
 (segment (start 97.4 54.3) (end 97.7 54.3) (width 0.5) (layer "B.Cu") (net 1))
 (segment (start 97.07 63.03) (end 97.56 62.54) (width 0.5) (layer "B.Cu") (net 1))
 (segment (start 96.61 63.03) (end 97.07 63.03) (width 0.5) (layer "B.Cu") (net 1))
 (segment (start 98.3798 58.0098) (end 98.35 57.98) (width 0.5) (layer "F.Cu") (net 9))
 (segment (start 98.3798 62.1) (end 98.3798 58.0098) (width 0.5) (layer "F.Cu") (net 9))
 (segment (start 102.91 56.22) (end 99.52 56.22) (width 0.5) (layer "B.Cu") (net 9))
 (segment (start 99.52 56.22) (end 98.35 57.39) (width 0.5) (layer "B.Cu") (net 9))
 (segment (start 103.075 62.54) (end 101.77 62.54) (width 0.5) (layer "B.Cu") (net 9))
 (segment (start 101.14 60.42) (end 101.09 60.37) (width 0.5) (layer "B.Cu") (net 9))
 (segment (start 102.91 58.55) (end 102.91 56.22) (width 0.5) (layer "B.Cu") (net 9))
 (segment (start 98.35 57.39) (end 98.35 57.98) (width 0.5) (layer "B.Cu") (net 9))
 (segment (start 101.09 60.37) (end 102.91 58.55) (width 0.5) (layer "B.Cu") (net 9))
 (segment (start 101.14 61.91) (end 101.14 60.42) (width 0.5) (layer "B.Cu") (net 9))
 (segment (start 101.77 62.54) (end 101.14 61.91) (width 0.5) (layer "B.Cu") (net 9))
 (segment (start 96.960257 65.33) (end 93.03 65.33) (width 0.3) (layer "F.Cu") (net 3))
 (segment (start 93.03 65.33) (end 91.98 64.28) (width 0.3) (layer "F.Cu") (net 3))
 (segment (start 101.520331 64.560331) (end 101.520331 64.570331) (width 0.3) (layer "F.Cu") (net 3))
 (segment (start 102.0625 65.1125) (end 103.44 65.1125) (width 0.3) (layer "F.Cu") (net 3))
 (segment (start 101.520331 64.570331) (end 102.0625 65.1125) (width 0.3) (layer "F.Cu") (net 3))
 (segment (start 101.520331 64.560331) (end 101.499669 64.560331) (width 0.3) (layer "F.Cu") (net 3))
 (segment (start 101.499669 64.560331) (end 100.669 65.391) (width 0.3) (layer "F.Cu") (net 3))
 (segment (start 97.021257 65.391) (end 96.960257 65.33) (width 0.3) (layer "F.Cu") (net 3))
 (segment (start 100.669 65.391) (end 97.021257 65.391) (width 0.3) (layer "F.Cu") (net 3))
 (via (at 101.520331 64.560331) (size 0.6) (drill 0.3) (layers "F.Cu" "B.Cu") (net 3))
 (segment (start 101.520331 64.560331) (end 102.166926 65.206926) (width 0.3) (layer "B.Cu") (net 3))
 (segment (start 102.948074 65.206926) (end 103.075 65.08) (width 0.3) (layer "B.Cu") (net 3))
 (segment (start 102.166926 65.206926) (end 102.948074 65.206926) (width 0.3) (layer "B.Cu") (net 3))
 (segment (start 96.121 64.479) (end 94.719 64.479) (width 0.5) (layer "B.Cu") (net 2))
 (segment (start 98.125 63.81) (end 96.79 63.81) (width 0.5) (layer "B.Cu") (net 2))
 (segment (start 96.79 63.81) (end 96.121 64.479) (width 0.5) (layer "B.Cu") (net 2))
 (segment (start 94.719 64.479) (end 91.98 61.74) (width 0.5) (layer "B.Cu") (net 2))
 (segment (start 95.8 58.3) (end 95.6 58.3) (width 0.3) (layer "B.Cu") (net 8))
 (segment (start 94.205 59.695) (end 94.07 59.83) (width 0.5) (layer "B.Cu") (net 8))
 (segment (start 94.07 59.83) (end 94.07 60.18) (width 0.5) (layer "B.Cu") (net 8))
 (segment (start 95.72 58.38) (end 95.8 58.3) (width 0.3) (layer "B.Cu") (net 8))
 (segment (start 95.6 58.3) (end 94.205 59.695) (width 0.5) (layer "B.Cu") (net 8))
 (segment (start 100.6 58.3) (end 100.8 58.3) (width 0.3) (layer "F.Cu") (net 10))
 (segment (start 98.92 60.18) (end 96.07 60.18) (width 0.5) (layer "B.Cu") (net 10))
 (segment (start 98.92 60.18) (end 100.8 58.3) (width 0.5) (layer "B.Cu") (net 10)))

